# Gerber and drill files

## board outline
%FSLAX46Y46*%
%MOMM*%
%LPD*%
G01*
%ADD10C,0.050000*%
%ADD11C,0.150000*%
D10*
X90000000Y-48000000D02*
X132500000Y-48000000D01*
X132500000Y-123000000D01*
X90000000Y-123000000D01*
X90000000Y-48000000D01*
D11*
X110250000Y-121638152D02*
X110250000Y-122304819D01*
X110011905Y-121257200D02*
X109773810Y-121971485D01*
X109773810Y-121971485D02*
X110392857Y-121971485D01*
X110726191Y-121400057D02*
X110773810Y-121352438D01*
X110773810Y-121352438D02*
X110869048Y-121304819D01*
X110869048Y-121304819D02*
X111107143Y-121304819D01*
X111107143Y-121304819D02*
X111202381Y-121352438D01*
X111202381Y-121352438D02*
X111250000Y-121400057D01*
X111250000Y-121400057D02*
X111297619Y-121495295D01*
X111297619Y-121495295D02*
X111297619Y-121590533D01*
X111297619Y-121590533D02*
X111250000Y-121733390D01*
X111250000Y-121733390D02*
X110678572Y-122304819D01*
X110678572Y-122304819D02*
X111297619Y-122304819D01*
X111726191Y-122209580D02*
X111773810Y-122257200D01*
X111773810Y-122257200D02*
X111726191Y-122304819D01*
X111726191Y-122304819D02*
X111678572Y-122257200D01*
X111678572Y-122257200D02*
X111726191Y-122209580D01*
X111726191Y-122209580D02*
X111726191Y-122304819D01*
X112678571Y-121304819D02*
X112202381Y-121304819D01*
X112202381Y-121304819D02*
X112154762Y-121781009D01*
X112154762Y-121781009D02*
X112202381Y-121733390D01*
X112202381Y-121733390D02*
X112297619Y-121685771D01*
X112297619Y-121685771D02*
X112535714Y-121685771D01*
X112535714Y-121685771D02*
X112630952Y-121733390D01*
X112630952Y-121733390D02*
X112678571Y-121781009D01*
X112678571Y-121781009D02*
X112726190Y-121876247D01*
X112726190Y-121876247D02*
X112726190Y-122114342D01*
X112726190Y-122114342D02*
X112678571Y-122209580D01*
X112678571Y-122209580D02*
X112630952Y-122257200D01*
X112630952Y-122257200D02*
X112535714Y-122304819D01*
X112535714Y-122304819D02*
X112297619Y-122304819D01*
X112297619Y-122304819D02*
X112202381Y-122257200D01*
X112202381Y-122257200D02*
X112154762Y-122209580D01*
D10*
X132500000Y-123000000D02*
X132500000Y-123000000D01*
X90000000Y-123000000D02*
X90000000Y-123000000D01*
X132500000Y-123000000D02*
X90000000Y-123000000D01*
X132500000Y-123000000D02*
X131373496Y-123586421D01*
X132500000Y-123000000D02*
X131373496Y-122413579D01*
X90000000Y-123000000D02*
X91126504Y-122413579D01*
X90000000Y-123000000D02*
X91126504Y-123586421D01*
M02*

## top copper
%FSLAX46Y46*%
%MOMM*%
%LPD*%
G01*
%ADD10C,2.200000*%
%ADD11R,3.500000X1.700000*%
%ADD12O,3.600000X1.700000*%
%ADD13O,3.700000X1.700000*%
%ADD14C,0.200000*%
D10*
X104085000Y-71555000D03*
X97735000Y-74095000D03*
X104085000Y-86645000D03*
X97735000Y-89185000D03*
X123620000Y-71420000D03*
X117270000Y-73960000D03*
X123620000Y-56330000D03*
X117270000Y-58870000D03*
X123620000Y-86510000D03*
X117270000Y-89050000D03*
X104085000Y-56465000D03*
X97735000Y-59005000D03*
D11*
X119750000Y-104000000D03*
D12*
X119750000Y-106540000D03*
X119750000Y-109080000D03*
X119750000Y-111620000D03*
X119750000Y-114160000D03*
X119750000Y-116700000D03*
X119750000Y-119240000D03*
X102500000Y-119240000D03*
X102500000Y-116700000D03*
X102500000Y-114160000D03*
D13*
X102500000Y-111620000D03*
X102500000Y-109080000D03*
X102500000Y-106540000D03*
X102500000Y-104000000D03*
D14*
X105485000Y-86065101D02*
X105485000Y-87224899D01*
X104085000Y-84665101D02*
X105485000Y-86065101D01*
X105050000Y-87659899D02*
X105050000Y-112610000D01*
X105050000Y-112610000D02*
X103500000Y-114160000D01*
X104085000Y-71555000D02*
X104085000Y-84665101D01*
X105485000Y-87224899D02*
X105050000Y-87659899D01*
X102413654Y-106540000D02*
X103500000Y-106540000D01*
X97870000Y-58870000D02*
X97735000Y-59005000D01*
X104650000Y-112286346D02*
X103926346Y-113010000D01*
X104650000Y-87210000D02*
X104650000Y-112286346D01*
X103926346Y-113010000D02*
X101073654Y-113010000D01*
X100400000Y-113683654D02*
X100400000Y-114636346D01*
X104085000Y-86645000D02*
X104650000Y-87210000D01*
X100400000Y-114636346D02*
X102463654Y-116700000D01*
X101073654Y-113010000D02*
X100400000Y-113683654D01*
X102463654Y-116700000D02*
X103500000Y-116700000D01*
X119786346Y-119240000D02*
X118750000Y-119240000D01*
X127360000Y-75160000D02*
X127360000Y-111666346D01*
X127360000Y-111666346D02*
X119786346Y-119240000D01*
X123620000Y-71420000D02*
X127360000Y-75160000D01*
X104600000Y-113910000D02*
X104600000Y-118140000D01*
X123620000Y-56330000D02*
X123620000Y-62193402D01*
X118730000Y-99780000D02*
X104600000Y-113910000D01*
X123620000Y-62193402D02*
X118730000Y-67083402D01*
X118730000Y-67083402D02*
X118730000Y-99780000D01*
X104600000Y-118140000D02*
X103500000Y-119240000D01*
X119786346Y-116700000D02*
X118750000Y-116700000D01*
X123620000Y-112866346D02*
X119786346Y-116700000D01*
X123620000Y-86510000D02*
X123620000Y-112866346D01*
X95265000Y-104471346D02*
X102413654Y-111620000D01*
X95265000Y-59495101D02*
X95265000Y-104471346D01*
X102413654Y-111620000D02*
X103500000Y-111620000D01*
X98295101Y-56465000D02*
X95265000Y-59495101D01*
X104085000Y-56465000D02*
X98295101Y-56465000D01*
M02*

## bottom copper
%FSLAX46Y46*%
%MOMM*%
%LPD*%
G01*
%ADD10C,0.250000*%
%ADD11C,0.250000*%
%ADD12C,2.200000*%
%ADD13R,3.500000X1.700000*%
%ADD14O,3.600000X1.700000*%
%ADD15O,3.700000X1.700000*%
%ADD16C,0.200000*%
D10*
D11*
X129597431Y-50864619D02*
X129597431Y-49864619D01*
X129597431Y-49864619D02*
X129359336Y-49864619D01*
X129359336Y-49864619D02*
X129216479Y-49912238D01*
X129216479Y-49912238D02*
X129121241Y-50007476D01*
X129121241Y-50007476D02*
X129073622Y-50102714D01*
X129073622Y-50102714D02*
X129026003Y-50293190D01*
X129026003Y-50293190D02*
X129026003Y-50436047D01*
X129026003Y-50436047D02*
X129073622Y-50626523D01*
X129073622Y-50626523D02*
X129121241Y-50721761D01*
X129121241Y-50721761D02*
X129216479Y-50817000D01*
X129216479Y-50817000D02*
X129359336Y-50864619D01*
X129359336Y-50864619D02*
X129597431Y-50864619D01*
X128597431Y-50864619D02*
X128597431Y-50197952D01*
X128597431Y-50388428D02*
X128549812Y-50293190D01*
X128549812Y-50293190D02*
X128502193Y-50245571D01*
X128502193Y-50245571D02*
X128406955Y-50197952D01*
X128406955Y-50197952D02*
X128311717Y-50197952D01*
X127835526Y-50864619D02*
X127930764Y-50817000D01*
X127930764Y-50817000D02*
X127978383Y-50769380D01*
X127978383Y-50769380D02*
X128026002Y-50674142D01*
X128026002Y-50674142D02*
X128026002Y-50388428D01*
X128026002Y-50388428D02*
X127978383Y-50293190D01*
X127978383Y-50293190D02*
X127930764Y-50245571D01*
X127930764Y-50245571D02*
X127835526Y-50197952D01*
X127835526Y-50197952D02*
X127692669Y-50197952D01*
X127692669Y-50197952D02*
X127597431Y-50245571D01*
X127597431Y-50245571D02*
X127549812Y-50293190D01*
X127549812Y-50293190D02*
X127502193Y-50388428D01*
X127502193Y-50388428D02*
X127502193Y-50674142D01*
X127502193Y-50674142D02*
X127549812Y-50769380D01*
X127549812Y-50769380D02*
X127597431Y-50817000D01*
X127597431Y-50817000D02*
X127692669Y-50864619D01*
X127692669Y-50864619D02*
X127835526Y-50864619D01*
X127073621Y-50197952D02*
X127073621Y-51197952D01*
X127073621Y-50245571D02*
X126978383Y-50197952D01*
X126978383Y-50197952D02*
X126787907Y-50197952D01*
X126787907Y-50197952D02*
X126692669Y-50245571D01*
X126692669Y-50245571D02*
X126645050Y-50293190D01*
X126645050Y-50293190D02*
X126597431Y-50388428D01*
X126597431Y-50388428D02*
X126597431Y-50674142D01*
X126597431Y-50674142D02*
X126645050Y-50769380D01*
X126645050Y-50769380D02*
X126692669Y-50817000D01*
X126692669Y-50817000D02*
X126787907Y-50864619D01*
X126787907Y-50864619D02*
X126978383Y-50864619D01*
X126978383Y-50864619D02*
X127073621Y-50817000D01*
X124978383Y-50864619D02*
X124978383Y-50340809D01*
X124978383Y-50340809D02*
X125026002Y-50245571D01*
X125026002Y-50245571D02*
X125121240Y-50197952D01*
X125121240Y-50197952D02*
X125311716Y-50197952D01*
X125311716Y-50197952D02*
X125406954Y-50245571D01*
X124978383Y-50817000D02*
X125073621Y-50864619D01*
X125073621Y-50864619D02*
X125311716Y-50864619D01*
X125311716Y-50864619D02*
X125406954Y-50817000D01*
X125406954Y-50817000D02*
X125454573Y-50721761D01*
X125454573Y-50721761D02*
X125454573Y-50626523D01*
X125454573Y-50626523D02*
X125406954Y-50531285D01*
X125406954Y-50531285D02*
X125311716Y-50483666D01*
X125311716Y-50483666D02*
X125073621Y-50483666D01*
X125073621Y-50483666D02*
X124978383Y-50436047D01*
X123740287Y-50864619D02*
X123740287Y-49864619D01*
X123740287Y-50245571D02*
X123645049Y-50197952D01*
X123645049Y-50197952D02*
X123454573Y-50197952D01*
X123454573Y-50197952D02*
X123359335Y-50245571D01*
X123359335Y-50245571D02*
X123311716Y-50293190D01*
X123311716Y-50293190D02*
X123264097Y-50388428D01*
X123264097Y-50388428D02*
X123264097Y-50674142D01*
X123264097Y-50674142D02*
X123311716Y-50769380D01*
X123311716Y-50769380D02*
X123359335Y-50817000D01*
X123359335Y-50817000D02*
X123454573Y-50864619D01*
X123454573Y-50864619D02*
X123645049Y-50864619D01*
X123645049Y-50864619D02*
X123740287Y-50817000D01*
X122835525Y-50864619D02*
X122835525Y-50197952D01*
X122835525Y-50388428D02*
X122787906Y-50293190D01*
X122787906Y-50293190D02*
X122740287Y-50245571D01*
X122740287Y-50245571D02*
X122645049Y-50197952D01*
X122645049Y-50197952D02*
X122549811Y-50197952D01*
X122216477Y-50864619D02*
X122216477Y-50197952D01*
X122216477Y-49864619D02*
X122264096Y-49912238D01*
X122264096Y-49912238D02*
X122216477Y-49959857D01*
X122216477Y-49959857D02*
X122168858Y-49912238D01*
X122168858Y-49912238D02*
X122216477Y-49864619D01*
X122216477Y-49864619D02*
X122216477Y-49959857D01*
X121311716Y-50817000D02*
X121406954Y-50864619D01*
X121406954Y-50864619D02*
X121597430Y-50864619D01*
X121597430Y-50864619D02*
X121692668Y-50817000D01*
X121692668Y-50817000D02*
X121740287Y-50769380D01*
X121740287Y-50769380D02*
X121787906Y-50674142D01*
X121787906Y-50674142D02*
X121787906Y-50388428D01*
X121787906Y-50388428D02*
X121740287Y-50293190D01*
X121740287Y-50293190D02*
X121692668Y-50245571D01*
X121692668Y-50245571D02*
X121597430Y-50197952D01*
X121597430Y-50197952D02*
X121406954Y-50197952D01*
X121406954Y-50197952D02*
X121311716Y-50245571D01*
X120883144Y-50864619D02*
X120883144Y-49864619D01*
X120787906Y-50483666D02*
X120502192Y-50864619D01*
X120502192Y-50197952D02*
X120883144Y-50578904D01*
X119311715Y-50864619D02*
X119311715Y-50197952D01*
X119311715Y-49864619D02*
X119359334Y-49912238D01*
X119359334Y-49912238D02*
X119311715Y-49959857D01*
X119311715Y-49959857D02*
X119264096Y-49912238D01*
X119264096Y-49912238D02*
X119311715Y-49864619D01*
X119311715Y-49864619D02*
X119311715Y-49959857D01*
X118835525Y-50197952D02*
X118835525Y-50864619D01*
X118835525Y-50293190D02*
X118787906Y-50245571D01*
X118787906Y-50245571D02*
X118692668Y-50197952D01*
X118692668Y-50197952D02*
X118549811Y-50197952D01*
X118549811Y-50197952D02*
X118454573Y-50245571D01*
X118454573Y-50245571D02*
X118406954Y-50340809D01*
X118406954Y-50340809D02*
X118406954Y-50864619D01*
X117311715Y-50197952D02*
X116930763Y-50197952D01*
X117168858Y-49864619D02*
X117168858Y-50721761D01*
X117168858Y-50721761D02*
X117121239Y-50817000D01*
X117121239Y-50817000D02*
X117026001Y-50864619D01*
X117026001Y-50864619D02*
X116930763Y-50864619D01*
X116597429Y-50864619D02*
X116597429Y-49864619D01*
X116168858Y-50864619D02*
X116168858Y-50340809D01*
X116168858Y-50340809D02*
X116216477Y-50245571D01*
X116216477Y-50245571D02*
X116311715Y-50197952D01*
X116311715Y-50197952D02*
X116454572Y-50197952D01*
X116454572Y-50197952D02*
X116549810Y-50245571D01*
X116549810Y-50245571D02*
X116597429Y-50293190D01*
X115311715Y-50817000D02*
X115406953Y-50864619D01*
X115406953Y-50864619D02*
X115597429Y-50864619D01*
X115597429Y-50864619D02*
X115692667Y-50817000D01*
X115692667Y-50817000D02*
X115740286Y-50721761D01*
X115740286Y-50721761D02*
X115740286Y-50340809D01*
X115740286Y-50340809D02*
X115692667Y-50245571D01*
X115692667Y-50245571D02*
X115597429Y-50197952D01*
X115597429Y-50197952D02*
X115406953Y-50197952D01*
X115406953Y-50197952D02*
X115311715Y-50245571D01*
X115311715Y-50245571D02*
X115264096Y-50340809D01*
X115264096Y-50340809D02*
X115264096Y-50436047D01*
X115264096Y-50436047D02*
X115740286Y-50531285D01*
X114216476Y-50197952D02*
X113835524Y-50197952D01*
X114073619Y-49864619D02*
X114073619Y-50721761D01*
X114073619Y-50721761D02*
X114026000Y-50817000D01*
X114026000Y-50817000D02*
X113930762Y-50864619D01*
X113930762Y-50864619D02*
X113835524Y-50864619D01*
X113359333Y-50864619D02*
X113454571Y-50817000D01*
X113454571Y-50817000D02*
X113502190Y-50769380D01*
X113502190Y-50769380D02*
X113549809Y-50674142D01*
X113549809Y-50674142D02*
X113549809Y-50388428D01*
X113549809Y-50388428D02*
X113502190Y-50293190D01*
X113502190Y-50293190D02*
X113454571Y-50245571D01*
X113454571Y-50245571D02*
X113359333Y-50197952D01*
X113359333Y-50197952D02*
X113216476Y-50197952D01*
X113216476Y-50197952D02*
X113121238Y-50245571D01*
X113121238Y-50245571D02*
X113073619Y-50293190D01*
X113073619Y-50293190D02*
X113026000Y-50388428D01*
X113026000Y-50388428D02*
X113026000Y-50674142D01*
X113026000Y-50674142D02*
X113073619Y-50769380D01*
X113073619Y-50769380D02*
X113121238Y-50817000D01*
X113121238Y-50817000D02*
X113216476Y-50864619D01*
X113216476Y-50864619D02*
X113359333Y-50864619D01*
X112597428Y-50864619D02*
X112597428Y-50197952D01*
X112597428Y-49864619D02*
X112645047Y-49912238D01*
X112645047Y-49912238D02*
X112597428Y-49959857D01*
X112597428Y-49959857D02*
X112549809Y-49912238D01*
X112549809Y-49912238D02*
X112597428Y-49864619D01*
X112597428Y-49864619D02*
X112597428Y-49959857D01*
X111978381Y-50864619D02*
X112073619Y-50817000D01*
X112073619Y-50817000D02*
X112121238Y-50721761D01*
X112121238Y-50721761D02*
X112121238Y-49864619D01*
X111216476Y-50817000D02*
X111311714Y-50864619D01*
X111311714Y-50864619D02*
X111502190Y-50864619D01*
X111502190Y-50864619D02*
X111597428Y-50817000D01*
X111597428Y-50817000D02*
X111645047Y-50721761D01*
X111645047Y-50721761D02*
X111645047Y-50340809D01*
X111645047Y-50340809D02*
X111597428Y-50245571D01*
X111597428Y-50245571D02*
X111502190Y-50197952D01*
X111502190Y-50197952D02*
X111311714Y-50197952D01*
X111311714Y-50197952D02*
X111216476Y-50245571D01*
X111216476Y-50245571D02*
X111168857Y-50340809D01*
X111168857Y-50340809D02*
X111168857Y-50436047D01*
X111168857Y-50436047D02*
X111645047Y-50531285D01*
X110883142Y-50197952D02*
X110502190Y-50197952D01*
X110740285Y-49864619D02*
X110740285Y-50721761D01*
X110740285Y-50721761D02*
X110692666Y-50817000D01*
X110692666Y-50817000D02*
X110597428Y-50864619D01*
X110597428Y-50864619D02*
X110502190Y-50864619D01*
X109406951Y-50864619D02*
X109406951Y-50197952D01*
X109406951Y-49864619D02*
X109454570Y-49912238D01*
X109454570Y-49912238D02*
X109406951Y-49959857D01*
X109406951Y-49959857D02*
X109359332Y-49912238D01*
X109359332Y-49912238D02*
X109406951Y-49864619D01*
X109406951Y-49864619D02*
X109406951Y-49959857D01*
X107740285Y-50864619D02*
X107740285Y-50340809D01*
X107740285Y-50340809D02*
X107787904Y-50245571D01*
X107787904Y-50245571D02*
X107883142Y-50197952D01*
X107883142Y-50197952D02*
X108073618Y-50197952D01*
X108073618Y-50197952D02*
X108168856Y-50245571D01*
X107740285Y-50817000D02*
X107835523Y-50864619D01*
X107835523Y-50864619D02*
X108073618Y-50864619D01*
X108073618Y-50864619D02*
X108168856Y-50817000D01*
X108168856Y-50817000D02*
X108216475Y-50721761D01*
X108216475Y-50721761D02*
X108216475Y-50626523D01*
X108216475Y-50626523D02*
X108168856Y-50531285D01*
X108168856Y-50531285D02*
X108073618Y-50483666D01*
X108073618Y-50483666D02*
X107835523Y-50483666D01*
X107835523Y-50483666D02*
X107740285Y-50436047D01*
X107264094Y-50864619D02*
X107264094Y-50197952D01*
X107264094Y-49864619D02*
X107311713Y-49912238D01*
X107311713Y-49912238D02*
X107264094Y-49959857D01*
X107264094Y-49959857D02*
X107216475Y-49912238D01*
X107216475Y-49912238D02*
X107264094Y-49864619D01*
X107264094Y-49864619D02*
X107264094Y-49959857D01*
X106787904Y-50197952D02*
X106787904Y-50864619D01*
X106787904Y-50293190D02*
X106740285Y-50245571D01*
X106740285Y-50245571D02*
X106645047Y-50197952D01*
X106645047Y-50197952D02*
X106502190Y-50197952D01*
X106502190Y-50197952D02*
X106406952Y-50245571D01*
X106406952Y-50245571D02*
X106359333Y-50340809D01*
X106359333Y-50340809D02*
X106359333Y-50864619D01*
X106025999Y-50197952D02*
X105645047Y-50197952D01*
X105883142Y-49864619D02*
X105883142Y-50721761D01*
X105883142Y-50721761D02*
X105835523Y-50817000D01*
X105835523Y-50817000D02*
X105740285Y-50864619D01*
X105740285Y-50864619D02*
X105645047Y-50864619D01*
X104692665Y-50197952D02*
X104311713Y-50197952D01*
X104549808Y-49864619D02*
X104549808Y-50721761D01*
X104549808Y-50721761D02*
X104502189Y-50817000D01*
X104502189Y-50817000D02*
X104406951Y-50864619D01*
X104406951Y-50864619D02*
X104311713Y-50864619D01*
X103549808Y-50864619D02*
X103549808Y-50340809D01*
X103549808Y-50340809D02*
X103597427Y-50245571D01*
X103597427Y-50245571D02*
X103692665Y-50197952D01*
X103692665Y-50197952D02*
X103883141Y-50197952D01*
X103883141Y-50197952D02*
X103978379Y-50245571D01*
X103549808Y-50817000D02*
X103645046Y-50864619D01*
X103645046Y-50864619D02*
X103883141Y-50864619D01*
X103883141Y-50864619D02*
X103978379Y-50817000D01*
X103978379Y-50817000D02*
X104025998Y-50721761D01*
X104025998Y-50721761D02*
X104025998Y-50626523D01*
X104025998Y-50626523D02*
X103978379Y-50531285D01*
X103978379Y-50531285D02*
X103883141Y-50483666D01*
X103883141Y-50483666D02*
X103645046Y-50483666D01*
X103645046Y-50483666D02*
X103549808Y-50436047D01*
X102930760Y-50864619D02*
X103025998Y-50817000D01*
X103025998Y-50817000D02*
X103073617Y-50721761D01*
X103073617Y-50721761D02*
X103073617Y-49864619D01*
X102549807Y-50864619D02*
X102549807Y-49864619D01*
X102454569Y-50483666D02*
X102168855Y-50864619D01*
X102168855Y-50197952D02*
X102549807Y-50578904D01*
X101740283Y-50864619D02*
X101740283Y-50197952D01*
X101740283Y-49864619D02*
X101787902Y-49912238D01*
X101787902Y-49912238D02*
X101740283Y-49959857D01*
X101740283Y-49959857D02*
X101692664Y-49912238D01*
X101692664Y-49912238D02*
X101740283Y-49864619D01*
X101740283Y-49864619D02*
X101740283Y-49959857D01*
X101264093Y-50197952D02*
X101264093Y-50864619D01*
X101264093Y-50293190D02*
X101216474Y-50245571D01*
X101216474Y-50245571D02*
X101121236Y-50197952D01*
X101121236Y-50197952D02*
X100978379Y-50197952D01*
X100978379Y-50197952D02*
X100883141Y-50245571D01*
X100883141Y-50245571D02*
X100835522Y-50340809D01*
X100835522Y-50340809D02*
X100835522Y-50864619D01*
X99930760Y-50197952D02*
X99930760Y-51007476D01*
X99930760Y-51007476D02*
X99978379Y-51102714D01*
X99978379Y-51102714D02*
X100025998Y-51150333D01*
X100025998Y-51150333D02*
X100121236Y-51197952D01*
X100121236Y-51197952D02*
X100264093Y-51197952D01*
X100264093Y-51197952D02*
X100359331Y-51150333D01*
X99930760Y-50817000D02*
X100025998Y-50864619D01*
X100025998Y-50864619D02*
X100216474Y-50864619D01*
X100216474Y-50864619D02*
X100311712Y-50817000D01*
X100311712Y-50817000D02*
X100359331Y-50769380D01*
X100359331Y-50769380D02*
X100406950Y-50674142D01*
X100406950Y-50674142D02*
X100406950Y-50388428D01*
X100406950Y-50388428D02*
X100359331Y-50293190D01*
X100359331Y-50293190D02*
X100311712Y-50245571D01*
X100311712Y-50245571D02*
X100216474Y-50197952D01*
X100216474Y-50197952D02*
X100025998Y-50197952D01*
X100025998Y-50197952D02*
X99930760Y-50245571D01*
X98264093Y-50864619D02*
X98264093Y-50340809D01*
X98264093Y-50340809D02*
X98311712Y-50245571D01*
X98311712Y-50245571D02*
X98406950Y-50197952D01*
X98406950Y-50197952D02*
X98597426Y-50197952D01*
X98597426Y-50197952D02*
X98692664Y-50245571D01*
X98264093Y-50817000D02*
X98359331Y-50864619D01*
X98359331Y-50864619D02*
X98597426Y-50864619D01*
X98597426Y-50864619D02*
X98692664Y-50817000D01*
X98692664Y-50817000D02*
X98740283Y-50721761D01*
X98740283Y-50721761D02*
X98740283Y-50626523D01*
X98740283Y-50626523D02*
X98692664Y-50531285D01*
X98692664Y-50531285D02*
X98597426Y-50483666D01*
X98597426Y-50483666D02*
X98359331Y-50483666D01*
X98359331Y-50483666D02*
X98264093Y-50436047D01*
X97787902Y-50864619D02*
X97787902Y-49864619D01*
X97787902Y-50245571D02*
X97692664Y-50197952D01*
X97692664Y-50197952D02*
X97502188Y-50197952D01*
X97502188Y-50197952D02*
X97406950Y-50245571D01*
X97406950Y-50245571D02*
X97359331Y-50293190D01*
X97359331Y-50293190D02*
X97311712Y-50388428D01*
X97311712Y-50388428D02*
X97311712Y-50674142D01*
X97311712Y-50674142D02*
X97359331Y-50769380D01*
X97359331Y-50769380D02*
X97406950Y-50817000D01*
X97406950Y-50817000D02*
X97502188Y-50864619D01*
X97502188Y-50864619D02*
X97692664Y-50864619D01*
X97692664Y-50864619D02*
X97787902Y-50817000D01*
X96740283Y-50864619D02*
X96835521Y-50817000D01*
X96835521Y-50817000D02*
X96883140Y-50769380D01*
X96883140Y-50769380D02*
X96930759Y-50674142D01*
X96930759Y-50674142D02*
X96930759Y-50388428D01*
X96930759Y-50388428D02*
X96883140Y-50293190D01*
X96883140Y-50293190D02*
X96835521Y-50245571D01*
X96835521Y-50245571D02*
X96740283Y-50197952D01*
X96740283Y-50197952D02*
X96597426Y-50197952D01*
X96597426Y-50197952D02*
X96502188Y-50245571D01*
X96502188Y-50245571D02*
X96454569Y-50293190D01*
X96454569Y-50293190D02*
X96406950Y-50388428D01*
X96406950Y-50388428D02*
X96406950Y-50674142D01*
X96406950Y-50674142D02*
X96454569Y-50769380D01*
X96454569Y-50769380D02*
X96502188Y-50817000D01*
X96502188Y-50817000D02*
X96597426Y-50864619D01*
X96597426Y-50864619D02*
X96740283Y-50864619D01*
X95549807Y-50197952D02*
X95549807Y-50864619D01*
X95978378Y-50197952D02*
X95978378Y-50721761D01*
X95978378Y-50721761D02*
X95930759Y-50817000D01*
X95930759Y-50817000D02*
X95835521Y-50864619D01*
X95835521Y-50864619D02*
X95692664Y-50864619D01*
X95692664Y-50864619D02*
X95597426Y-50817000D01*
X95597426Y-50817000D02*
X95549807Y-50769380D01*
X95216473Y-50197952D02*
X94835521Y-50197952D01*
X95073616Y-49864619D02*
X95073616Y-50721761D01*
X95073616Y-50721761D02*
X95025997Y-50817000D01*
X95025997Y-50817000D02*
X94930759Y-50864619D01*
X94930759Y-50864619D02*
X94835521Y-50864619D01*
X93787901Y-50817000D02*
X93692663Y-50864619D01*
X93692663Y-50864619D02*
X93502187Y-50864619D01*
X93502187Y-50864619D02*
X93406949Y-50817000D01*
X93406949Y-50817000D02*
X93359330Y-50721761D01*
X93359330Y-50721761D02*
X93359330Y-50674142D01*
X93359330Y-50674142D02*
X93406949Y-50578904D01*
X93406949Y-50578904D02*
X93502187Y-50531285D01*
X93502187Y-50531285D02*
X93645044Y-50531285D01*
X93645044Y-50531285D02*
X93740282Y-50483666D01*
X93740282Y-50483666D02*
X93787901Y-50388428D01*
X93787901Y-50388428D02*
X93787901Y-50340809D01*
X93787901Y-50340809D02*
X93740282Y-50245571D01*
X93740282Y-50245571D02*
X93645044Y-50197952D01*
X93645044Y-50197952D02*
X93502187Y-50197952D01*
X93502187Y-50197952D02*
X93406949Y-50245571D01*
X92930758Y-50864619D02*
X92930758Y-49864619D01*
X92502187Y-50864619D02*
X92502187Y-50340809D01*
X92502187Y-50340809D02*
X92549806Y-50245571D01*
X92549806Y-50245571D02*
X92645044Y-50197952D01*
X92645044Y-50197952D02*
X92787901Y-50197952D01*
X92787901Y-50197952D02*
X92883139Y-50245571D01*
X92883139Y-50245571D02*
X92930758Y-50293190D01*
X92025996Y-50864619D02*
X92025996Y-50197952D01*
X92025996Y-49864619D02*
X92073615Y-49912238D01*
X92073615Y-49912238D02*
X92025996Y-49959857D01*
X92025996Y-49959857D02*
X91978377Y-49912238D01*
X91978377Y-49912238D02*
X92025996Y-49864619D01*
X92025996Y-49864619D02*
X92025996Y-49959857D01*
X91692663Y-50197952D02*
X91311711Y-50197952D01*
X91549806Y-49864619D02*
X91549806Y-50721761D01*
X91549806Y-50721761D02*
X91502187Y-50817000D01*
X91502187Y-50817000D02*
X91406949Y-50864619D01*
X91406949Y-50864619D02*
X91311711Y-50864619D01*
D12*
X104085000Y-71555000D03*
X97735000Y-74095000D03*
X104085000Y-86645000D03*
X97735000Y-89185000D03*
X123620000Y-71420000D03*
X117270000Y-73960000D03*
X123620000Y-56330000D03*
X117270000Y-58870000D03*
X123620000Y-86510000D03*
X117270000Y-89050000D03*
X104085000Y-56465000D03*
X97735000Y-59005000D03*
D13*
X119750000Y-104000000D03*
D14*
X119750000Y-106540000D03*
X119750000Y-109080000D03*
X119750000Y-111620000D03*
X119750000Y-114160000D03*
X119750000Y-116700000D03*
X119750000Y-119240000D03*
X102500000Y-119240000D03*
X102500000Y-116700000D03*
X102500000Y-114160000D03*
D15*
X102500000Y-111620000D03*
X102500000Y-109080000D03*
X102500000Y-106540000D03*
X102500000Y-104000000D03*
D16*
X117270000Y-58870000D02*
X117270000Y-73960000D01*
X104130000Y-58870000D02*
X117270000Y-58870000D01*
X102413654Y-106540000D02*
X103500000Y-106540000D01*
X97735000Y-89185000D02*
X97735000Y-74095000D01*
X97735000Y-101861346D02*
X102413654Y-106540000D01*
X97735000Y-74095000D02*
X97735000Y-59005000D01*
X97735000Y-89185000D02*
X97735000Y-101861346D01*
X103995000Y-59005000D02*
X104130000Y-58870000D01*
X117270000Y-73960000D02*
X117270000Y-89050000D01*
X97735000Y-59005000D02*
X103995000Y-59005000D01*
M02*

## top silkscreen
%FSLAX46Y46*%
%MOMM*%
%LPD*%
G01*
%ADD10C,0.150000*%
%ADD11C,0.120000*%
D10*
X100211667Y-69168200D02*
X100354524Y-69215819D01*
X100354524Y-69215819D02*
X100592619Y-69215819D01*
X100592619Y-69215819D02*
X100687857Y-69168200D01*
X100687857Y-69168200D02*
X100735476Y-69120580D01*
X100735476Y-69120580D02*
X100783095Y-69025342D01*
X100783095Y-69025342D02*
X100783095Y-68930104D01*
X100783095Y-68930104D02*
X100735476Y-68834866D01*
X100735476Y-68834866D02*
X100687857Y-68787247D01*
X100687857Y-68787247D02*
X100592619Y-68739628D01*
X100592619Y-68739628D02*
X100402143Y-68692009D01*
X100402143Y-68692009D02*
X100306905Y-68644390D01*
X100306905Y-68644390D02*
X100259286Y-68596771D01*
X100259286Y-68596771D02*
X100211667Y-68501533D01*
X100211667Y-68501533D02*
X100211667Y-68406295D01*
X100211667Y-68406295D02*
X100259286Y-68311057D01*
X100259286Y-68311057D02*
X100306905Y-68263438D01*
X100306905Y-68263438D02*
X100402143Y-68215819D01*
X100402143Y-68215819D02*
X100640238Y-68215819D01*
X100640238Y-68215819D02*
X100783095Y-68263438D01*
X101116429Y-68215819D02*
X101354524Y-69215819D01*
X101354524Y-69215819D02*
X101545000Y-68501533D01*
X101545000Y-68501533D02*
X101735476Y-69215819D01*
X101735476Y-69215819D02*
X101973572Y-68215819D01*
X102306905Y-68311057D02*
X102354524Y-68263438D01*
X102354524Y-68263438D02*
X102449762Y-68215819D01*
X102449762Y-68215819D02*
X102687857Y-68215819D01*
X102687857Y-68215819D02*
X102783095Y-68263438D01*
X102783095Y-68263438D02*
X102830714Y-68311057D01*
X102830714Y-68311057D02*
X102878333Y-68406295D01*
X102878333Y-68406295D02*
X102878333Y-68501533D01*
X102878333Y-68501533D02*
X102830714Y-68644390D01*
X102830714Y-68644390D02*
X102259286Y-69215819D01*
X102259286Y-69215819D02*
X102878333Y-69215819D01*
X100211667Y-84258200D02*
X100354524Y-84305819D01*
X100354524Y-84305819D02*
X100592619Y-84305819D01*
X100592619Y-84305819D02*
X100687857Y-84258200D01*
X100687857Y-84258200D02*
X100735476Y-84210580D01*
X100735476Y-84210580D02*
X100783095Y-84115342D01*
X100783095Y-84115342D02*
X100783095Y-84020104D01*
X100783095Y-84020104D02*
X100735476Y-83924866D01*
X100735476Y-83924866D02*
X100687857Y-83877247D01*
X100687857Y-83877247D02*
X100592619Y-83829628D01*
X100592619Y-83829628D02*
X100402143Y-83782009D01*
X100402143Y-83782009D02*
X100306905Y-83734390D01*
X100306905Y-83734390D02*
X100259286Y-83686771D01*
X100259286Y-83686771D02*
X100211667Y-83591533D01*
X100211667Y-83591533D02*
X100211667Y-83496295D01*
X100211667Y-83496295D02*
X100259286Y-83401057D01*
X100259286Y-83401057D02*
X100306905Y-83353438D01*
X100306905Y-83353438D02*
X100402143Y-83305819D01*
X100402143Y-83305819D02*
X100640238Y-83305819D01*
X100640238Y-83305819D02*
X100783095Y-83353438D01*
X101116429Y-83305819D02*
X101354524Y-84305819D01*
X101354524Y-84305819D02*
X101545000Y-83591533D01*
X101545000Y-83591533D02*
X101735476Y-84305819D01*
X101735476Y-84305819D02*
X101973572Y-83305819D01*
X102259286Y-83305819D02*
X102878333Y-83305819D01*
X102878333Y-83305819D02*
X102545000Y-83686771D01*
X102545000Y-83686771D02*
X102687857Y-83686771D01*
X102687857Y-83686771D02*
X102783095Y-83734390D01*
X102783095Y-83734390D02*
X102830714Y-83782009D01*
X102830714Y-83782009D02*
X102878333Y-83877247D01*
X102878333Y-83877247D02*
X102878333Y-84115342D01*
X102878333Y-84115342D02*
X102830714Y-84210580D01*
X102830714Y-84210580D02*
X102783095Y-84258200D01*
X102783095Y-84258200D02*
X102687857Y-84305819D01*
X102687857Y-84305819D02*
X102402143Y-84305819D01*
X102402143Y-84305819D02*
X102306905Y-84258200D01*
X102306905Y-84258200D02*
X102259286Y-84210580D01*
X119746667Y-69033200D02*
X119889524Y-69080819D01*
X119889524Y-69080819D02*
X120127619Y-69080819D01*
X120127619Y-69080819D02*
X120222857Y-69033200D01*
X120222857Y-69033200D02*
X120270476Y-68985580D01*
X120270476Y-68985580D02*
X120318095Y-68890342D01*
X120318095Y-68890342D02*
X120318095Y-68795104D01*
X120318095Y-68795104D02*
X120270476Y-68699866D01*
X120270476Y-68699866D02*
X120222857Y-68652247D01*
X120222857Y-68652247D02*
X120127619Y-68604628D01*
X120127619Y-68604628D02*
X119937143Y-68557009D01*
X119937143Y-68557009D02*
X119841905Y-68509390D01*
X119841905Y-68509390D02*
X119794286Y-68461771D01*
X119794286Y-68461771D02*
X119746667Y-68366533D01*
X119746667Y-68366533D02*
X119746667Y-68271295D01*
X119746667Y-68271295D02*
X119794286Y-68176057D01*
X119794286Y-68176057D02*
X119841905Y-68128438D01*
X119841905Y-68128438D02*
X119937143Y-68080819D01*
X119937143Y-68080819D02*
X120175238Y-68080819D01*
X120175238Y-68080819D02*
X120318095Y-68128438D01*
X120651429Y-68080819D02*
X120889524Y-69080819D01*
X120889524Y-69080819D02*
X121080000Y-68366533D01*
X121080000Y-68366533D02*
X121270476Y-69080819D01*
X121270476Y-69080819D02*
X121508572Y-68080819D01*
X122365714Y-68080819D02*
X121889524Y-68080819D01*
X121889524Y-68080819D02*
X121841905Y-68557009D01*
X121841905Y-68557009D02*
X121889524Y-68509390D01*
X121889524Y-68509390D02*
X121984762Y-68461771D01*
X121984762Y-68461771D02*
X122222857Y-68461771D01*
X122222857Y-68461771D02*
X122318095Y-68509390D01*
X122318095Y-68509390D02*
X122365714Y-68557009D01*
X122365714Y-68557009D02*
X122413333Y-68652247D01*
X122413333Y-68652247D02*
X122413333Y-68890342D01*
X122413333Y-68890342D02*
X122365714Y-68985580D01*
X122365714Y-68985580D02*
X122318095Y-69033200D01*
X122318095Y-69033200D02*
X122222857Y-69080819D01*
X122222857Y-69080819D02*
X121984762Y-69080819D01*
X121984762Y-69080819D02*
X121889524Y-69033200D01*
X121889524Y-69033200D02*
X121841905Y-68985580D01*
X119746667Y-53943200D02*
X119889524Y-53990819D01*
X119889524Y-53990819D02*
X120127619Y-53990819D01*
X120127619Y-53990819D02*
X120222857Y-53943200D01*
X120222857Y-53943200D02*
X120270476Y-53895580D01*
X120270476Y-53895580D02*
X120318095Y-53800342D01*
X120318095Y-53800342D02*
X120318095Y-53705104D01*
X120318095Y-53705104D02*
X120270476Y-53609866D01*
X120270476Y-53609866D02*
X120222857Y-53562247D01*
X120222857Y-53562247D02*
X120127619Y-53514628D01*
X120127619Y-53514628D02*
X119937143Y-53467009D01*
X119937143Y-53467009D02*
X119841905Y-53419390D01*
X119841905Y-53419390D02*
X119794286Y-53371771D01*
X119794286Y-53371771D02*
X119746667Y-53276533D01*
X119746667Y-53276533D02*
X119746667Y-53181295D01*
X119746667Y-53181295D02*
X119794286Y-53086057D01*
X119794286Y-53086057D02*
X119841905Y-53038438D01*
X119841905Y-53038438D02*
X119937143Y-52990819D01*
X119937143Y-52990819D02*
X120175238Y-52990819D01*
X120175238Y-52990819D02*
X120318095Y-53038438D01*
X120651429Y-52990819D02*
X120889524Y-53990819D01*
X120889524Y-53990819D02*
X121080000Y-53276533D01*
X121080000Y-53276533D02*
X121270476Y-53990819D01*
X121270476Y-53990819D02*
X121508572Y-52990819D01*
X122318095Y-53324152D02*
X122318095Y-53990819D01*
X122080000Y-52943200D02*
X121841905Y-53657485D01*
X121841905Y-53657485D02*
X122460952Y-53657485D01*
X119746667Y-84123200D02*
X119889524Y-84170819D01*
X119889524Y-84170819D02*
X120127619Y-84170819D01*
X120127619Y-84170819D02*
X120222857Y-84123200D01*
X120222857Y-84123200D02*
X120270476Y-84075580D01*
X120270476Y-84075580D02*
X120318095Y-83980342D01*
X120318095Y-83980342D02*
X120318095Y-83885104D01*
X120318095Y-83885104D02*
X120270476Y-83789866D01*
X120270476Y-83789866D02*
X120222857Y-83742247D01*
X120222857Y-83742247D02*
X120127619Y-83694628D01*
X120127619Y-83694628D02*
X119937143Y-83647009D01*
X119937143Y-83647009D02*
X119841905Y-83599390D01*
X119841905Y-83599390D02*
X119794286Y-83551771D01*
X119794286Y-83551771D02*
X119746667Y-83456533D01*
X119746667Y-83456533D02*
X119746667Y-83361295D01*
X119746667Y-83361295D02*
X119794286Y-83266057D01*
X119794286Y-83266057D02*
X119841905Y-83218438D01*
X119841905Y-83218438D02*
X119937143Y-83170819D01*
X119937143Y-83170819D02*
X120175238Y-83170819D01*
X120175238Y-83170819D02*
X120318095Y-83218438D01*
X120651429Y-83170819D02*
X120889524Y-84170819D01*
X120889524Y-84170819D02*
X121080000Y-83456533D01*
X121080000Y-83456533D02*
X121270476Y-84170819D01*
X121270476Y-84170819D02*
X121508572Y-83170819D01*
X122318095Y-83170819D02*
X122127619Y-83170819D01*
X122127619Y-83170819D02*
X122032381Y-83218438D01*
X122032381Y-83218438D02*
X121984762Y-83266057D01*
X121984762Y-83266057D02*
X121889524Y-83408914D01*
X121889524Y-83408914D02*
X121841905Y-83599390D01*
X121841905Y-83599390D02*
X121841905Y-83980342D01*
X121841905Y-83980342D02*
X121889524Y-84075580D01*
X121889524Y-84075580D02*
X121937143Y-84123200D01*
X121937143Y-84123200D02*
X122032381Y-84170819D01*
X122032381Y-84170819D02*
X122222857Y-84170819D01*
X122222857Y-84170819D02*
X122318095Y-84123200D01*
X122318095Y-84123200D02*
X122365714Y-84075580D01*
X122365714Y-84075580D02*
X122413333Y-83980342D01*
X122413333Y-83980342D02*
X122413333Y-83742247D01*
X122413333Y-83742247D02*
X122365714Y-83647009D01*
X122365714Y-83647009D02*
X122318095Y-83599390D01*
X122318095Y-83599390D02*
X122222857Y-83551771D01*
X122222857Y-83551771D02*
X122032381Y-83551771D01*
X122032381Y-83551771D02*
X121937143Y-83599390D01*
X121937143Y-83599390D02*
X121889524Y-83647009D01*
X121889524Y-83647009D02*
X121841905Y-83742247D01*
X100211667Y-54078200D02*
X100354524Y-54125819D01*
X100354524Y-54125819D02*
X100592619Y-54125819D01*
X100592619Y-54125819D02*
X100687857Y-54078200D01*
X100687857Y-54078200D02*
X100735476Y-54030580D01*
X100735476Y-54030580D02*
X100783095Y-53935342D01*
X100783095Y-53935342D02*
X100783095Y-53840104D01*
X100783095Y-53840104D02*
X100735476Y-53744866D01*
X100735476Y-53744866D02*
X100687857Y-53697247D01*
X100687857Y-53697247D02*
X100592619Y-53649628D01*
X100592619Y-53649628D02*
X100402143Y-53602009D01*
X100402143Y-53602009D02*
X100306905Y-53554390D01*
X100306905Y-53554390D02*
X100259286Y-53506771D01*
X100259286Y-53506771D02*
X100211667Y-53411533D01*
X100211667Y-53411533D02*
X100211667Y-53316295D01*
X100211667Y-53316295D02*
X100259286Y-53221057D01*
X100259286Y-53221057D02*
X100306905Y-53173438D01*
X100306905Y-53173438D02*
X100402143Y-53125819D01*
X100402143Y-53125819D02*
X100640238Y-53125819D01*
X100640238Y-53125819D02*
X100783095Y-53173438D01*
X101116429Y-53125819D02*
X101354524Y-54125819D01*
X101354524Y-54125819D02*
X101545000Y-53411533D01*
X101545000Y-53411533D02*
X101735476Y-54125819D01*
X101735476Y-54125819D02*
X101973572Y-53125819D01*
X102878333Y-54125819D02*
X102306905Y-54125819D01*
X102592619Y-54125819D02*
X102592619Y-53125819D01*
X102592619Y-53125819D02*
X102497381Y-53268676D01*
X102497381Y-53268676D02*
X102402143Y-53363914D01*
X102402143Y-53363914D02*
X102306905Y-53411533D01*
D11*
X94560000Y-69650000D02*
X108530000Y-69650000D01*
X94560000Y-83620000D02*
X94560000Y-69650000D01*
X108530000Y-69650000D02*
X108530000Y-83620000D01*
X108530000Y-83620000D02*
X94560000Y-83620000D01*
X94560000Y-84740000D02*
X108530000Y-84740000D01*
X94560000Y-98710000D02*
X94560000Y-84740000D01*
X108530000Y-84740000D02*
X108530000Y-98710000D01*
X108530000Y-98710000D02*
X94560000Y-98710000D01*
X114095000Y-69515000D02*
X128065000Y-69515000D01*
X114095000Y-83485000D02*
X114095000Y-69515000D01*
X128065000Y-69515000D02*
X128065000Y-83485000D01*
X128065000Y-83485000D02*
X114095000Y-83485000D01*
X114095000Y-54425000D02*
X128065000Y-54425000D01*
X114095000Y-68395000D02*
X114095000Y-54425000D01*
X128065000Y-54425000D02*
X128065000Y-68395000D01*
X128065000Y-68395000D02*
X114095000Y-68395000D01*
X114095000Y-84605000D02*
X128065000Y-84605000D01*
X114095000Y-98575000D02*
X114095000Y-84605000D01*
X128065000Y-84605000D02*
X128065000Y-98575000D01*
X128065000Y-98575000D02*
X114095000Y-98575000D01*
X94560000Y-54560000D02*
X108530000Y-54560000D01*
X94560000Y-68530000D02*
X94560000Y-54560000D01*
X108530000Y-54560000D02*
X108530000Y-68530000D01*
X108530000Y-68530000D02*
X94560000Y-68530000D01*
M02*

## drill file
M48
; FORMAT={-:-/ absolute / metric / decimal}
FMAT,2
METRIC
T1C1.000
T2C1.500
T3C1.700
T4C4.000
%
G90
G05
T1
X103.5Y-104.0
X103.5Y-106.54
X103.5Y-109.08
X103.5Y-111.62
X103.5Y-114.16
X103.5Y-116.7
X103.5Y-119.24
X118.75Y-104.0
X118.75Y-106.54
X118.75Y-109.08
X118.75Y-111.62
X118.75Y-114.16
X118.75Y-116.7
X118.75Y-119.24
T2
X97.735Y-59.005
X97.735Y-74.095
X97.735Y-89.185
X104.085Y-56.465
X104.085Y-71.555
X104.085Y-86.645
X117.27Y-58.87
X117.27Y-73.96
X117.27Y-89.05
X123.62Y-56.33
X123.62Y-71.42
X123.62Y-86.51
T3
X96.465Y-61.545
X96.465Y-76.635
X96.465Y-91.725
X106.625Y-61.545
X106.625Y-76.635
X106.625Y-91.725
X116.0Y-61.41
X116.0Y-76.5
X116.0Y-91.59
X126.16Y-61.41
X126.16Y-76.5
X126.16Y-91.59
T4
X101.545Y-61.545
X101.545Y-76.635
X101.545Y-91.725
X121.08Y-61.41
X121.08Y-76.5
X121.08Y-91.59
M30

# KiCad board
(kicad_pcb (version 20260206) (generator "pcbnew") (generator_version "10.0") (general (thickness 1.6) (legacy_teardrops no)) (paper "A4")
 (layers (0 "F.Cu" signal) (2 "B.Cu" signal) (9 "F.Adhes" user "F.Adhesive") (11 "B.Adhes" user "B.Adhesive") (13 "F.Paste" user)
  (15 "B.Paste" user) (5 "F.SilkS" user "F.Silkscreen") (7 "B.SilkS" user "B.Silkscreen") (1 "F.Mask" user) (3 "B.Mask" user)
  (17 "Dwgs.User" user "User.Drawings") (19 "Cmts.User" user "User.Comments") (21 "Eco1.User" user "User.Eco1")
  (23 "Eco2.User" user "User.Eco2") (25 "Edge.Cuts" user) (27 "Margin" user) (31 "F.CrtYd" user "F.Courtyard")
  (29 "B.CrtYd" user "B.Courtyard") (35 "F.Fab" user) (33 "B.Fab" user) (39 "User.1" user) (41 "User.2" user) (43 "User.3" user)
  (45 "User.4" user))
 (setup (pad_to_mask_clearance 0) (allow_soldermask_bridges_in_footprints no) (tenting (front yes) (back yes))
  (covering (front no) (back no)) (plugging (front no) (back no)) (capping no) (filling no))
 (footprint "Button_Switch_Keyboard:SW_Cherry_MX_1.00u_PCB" (layer "F.Cu") (at 104.085 71.555)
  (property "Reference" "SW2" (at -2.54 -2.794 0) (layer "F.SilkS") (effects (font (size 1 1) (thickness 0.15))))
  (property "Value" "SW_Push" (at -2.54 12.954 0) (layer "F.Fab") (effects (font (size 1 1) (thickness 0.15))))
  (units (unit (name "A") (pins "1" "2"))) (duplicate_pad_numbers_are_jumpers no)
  (fp_line (start -9.525 -1.905) (end 4.445 -1.905) (stroke (width 0.12) (type solid)) (layer "F.SilkS"))
  (fp_line (start -9.525 12.065) (end -9.525 -1.905) (stroke (width 0.12) (type solid)) (layer "F.SilkS"))
  (fp_line (start 4.445 -1.905) (end 4.445 12.065) (stroke (width 0.12) (type solid)) (layer "F.SilkS"))
  (fp_line (start 4.445 12.065) (end -9.525 12.065) (stroke (width 0.12) (type solid)) (layer "F.SilkS"))
  (pad "" np_thru_hole circle (at -7.62 5.08) (size 1.7 1.7) (drill 1.7) (layers "*.Cu" "*.Mask"))
  (pad "" np_thru_hole circle (at -2.54 5.08) (size 4 4) (drill 4) (layers "*.Cu" "*.Mask"))
  (pad "" np_thru_hole circle (at 2.54 5.08) (size 1.7 1.7) (drill 1.7) (layers "*.Cu" "*.Mask"))
  (pad "1" thru_hole circle (at 0 0) (size 2.2 2.2) (drill 1.5) (layers "*.Cu" "*.Mask") (remove_unused_layers no)
   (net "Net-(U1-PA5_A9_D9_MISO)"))
  (pad "2" thru_hole circle (at -6.35 2.54) (size 2.2 2.2) (drill 1.5) (layers "*.Cu" "*.Mask") (remove_unused_layers no) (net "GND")))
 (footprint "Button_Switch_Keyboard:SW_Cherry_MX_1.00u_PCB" (layer "F.Cu") (at 104.085 86.645)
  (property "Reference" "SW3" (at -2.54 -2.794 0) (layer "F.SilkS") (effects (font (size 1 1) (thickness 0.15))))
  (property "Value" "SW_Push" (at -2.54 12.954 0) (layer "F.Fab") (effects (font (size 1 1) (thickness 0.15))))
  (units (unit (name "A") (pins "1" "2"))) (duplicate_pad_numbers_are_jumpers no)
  (fp_line (start -9.525 -1.905) (end 4.445 -1.905) (stroke (width 0.12) (type solid)) (layer "F.SilkS"))
  (fp_line (start -9.525 12.065) (end -9.525 -1.905) (stroke (width 0.12) (type solid)) (layer "F.SilkS"))
  (fp_line (start 4.445 -1.905) (end 4.445 12.065) (stroke (width 0.12) (type solid)) (layer "F.SilkS"))
  (fp_line (start 4.445 12.065) (end -9.525 12.065) (stroke (width 0.12) (type solid)) (layer "F.SilkS"))
  (pad "" np_thru_hole circle (at -7.62 5.08) (size 1.7 1.7) (drill 1.7) (layers "*.Cu" "*.Mask"))
  (pad "" np_thru_hole circle (at -2.54 5.08) (size 4 4) (drill 4) (layers "*.Cu" "*.Mask"))
  (pad "" np_thru_hole circle (at 2.54 5.08) (size 1.7 1.7) (drill 1.7) (layers "*.Cu" "*.Mask"))
  (pad "1" thru_hole circle (at 0 0) (size 2.2 2.2) (drill 1.5) (layers "*.Cu" "*.Mask") (remove_unused_layers no)
   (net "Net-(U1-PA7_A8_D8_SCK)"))
  (pad "2" thru_hole circle (at -6.35 2.54) (size 2.2 2.2) (drill 1.5) (layers "*.Cu" "*.Mask") (remove_unused_layers no) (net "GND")))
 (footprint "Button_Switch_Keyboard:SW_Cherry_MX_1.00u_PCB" (layer "F.Cu") (at 123.62 71.42)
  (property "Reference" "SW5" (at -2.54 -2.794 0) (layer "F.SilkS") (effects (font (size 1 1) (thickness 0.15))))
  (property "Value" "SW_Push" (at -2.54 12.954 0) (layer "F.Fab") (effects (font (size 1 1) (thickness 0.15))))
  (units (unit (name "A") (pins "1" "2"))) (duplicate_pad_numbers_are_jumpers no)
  (fp_line (start -9.525 -1.905) (end 4.445 -1.905) (stroke (width 0.12) (type solid)) (layer "F.SilkS"))
  (fp_line (start -9.525 12.065) (end -9.525 -1.905) (stroke (width 0.12) (type solid)) (layer "F.SilkS"))
  (fp_line (start 4.445 -1.905) (end 4.445 12.065) (stroke (width 0.12) (type solid)) (layer "F.SilkS"))
  (fp_line (start 4.445 12.065) (end -9.525 12.065) (stroke (width 0.12) (type solid)) (layer "F.SilkS"))
  (pad "" np_thru_hole circle (at -7.62 5.08) (size 1.7 1.7) (drill 1.7) (layers "*.Cu" "*.Mask"))
  (pad "" np_thru_hole circle (at -2.54 5.08) (size 4 4) (drill 4) (layers "*.Cu" "*.Mask"))
  (pad "" np_thru_hole circle (at 2.54 5.08) (size 1.7 1.7) (drill 1.7) (layers "*.Cu" "*.Mask"))
  (pad "1" thru_hole circle (at 0 0) (size 2.2 2.2) (drill 1.5) (layers "*.Cu" "*.Mask") (remove_unused_layers no)
   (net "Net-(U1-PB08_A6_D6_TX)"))
  (pad "2" thru_hole circle (at -6.35 2.54) (size 2.2 2.2) (drill 1.5) (layers "*.Cu" "*.Mask") (remove_unused_layers no) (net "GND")))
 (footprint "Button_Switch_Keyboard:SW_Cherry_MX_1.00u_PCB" (layer "F.Cu") (at 123.62 56.33)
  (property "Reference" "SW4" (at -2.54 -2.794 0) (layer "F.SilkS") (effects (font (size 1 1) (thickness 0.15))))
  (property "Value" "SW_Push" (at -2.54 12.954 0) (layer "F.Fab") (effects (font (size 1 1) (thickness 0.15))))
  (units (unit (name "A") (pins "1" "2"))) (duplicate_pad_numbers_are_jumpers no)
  (fp_line (start -9.525 -1.905) (end 4.445 -1.905) (stroke (width 0.12) (type solid)) (layer "F.SilkS"))
  (fp_line (start -9.525 12.065) (end -9.525 -1.905) (stroke (width 0.12) (type solid)) (layer "F.SilkS"))
  (fp_line (start 4.445 -1.905) (end 4.445 12.065) (stroke (width 0.12) (type solid)) (layer "F.SilkS"))
  (fp_line (start 4.445 12.065) (end -9.525 12.065) (stroke (width 0.12) (type solid)) (layer "F.SilkS"))
  (pad "" np_thru_hole circle (at -7.62 5.08) (size 1.7 1.7) (drill 1.7) (layers "*.Cu" "*.Mask"))
  (pad "" np_thru_hole circle (at -2.54 5.08) (size 4 4) (drill 4) (layers "*.Cu" "*.Mask"))
  (pad "" np_thru_hole circle (at 2.54 5.08) (size 1.7 1.7) (drill 1.7) (layers "*.Cu" "*.Mask"))
  (pad "1" thru_hole circle (at 0 0) (size 2.2 2.2) (drill 1.5) (layers "*.Cu" "*.Mask") (remove_unused_layers no)
   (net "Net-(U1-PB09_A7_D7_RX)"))
  (pad "2" thru_hole circle (at -6.35 2.54) (size 2.2 2.2) (drill 1.5) (layers "*.Cu" "*.Mask") (remove_unused_layers no) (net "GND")))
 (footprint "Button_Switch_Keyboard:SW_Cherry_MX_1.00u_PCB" (layer "F.Cu") (at 123.62 86.51)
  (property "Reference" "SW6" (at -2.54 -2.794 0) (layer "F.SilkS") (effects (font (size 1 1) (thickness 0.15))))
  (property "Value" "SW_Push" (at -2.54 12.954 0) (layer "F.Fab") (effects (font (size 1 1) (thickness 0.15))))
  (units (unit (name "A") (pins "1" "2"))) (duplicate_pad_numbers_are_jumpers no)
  (fp_line (start -9.525 -1.905) (end 4.445 -1.905) (stroke (width 0.12) (type solid)) (layer "F.SilkS"))
  (fp_line (start -9.525 12.065) (end -9.525 -1.905) (stroke (width 0.12) (type solid)) (layer "F.SilkS"))
  (fp_line (start 4.445 -1.905) (end 4.445 12.065) (stroke (width 0.12) (type solid)) (layer "F.SilkS"))
  (fp_line (start 4.445 12.065) (end -9.525 12.065) (stroke (width 0.12) (type solid)) (layer "F.SilkS"))
  (pad "" np_thru_hole circle (at -7.62 5.08) (size 1.7 1.7) (drill 1.7) (layers "*.Cu" "*.Mask"))
  (pad "" np_thru_hole circle (at -2.54 5.08) (size 4 4) (drill 4) (layers "*.Cu" "*.Mask"))
  (pad "" np_thru_hole circle (at 2.54 5.08) (size 1.7 1.7) (drill 1.7) (layers "*.Cu" "*.Mask"))
  (pad "1" thru_hole circle (at 0 0) (size 2.2 2.2) (drill 1.5) (layers "*.Cu" "*.Mask") (remove_unused_layers no)
   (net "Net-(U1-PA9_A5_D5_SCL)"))
  (pad "2" thru_hole circle (at -6.35 2.54) (size 2.2 2.2) (drill 1.5) (layers "*.Cu" "*.Mask") (remove_unused_layers no) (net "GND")))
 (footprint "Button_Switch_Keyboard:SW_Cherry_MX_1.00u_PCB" (layer "F.Cu") (at 104.085 56.465)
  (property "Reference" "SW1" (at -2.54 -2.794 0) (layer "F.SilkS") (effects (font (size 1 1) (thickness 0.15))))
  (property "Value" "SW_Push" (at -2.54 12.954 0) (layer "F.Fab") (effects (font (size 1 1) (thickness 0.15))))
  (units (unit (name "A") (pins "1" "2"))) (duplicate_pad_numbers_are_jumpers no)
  (fp_line (start -9.525 -1.905) (end 4.445 -1.905) (stroke (width 0.12) (type solid)) (layer "F.SilkS"))
  (fp_line (start -9.525 12.065) (end -9.525 -1.905) (stroke (width 0.12) (type solid)) (layer "F.SilkS"))
  (fp_line (start 4.445 -1.905) (end 4.445 12.065) (stroke (width 0.12) (type solid)) (layer "F.SilkS"))
  (fp_line (start 4.445 12.065) (end -9.525 12.065) (stroke (width 0.12) (type solid)) (layer "F.SilkS"))
  (pad "" np_thru_hole circle (at -7.62 5.08) (size 1.7 1.7) (drill 1.7) (layers "*.Cu" "*.Mask"))
  (pad "" np_thru_hole circle (at -2.54 5.08) (size 4 4) (drill 4) (layers "*.Cu" "*.Mask"))
  (pad "" np_thru_hole circle (at 2.54 5.08) (size 1.7 1.7) (drill 1.7) (layers "*.Cu" "*.Mask"))
  (pad "1" thru_hole circle (at 0 0) (size 2.2 2.2) (drill 1.5) (layers "*.Cu" "*.Mask") (remove_unused_layers no)
   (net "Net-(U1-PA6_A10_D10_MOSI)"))
  (pad "2" thru_hole circle (at -6.35 2.54) (size 2.2 2.2) (drill 1.5) (layers "*.Cu" "*.Mask") (remove_unused_layers no) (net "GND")))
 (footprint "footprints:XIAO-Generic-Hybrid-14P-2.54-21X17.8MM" (layer "B.Cu") (at 111.125 111.62 180)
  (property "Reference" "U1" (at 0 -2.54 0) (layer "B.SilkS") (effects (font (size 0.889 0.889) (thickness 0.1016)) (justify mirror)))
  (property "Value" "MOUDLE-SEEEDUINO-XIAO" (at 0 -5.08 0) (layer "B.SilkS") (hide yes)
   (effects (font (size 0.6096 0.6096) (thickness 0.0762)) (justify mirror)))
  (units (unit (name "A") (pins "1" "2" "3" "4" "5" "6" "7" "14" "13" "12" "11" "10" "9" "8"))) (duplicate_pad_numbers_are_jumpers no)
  (pad "1" thru_hole rect (at -7.625 7.62 180) (size 3.5 1.7) (drill 1 (offset -1 0)) (layers "*.Cu" "*.Mask") (remove_unused_layers no)
   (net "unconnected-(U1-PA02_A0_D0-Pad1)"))
  (pad "2" thru_hole oval (at -7.625 5.08 180) (size 3.6 1.7) (drill 1 (offset -1 0)) (layers "*.Cu" "*.Mask") (remove_unused_layers no)
   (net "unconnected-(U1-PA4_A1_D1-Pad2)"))
  (pad "3" thru_hole oval (at -7.625 2.54 180) (size 3.6 1.7) (drill 1 (offset -1 0)) (layers "*.Cu" "*.Mask") (remove_unused_layers no)
   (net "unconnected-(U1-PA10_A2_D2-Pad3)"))
  (pad "4" thru_hole oval (at -7.625 0 180) (size 3.6 1.7) (drill 1 (offset -1 0)) (layers "*.Cu" "*.Mask") (remove_unused_layers no)
   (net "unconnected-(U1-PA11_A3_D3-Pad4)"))
  (pad "5" thru_hole oval (at -7.625 -2.54 180) (size 3.6 1.7) (drill 1 (offset -1 0)) (layers "*.Cu" "*.Mask") (remove_unused_layers no)
   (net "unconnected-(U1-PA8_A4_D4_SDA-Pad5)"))
  (pad "6" thru_hole oval (at -7.625 -5.08) (size 3.6 1.7) (drill 1 (offset 1 0)) (layers "*.Cu" "*.Mask") (remove_unused_layers no)
   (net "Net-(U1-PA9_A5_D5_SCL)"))
  (pad "7" thru_hole oval (at -7.625 -7.62 180) (size 3.6 1.7) (drill 1 (offset -1 0)) (layers "*.Cu" "*.Mask") (remove_unused_layers no)
   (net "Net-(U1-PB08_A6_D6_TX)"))
  (pad "8" thru_hole oval (at 7.625 -7.62 180) (size 3.6 1.7) (drill 1 (offset 1 0)) (layers "*.Cu" "*.Mask") (remove_unused_layers no)
   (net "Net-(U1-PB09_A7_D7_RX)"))
  (pad "9" thru_hole oval (at 7.625 -5.08 180) (size 3.6 1.7) (drill 1 (offset 1 0)) (layers "*.Cu" "*.Mask") (remove_unused_layers no)
   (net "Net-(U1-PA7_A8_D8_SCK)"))
  (pad "10" thru_hole oval (at 7.625 -2.54 180) (size 3.6 1.7) (drill 1 (offset 1 0)) (layers "*.Cu" "*.Mask") (remove_unused_layers no)
   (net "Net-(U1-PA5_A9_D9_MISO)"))
  (pad "11" thru_hole oval (at 7.625 0 180) (size 3.7 1.7) (drill 1 (offset 1 0)) (layers "*.Cu" "*.Mask") (remove_unused_layers no)
   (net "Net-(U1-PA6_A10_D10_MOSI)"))
  (pad "12" thru_hole oval (at 7.625 2.54 180) (size 3.7 1.7) (drill 1 (offset 1 0)) (layers "*.Cu" "*.Mask") (remove_unused_layers no)
   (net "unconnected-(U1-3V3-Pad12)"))
  (pad "13" thru_hole oval (at 7.625 5.08 180) (size 3.7 1.7) (drill 1 (offset 1 0)) (layers "*.Cu" "*.Mask") (remove_unused_layers no)
   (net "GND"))
  (pad "14" thru_hole oval (at 7.625 7.62 180) (size 3.7 1.7) (drill 1 (offset 1 0)) (layers "*.Cu" "*.Mask") (remove_unused_layers no)
   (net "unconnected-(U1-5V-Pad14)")))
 (gr_rect (start 90 48) (end 132.5 123) (stroke (width 0.05) (type default)) (fill no) (layer "Edge.Cuts"))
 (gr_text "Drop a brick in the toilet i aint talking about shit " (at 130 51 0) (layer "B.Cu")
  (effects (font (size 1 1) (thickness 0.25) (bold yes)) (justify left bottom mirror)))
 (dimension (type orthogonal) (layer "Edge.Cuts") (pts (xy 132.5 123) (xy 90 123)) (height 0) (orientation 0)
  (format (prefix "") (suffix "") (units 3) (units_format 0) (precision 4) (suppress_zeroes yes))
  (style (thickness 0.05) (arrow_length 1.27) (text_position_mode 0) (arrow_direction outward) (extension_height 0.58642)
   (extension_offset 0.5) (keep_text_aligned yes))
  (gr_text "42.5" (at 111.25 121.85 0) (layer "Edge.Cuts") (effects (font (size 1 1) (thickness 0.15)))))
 (segment (start 105.485 86.065101) (end 105.485 87.224899) (width 0.2) (layer "F.Cu") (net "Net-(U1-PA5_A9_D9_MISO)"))
 (segment (start 104.085 84.665101) (end 105.485 86.065101) (width 0.2) (layer "F.Cu") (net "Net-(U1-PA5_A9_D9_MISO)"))
 (segment (start 105.05 87.659899) (end 105.05 112.61) (width 0.2) (layer "F.Cu") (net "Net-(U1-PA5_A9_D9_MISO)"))
 (segment (start 105.05 112.61) (end 103.5 114.16) (width 0.2) (layer "F.Cu") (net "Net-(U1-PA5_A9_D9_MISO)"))
 (segment (start 104.085 71.555) (end 104.085 84.665101) (width 0.2) (layer "F.Cu") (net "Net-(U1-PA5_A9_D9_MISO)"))
 (segment (start 105.485 87.224899) (end 105.05 87.659899) (width 0.2) (layer "F.Cu") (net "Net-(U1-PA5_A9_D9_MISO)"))
 (segment (start 102.413654 106.54) (end 103.5 106.54) (width 0.2) (layer "F.Cu") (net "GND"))
 (segment (start 97.87 58.87) (end 97.735 59.005) (width 0.2) (layer "F.Cu") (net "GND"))
 (segment (start 117.27 58.87) (end 117.27 73.96) (width 0.2) (layer "B.Cu") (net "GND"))
 (segment (start 104.13 58.87) (end 117.27 58.87) (width 0.2) (layer "B.Cu") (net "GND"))
 (segment (start 102.413654 106.54) (end 103.5 106.54) (width 0.2) (layer "B.Cu") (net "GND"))
 (segment (start 97.735 89.185) (end 97.735 74.095) (width 0.2) (layer "B.Cu") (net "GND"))
 (segment (start 97.735 101.861346) (end 102.413654 106.54) (width 0.2) (layer "B.Cu") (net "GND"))
 (segment (start 97.735 74.095) (end 97.735 59.005) (width 0.2) (layer "B.Cu") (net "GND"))
 (segment (start 97.735 89.185) (end 97.735 101.861346) (width 0.2) (layer "B.Cu") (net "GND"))
 (segment (start 103.995 59.005) (end 104.13 58.87) (width 0.2) (layer "B.Cu") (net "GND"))
 (segment (start 117.27 73.96) (end 117.27 89.05) (width 0.2) (layer "B.Cu") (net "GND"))
 (segment (start 97.735 59.005) (end 103.995 59.005) (width 0.2) (layer "B.Cu") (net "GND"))
 (segment (start 104.65 112.286346) (end 103.926346 113.01) (width 0.2) (layer "F.Cu") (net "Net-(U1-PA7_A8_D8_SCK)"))
 (segment (start 104.65 87.21) (end 104.65 112.286346) (width 0.2) (layer "F.Cu") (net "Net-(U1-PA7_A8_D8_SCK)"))
 (segment (start 103.926346 113.01) (end 101.073654 113.01) (width 0.2) (layer "F.Cu") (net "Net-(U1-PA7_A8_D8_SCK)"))
 (segment (start 100.4 113.683654) (end 100.4 114.636346) (width 0.2) (layer "F.Cu") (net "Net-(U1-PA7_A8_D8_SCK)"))
 (segment (start 104.085 86.645) (end 104.65 87.21) (width 0.2) (layer "F.Cu") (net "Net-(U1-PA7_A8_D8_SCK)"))
 (segment (start 100.4 114.636346) (end 102.463654 116.7) (width 0.2) (layer "F.Cu") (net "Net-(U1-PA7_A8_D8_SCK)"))
 (segment (start 101.073654 113.01) (end 100.4 113.683654) (width 0.2) (layer "F.Cu") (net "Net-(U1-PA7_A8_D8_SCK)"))
 (segment (start 102.463654 116.7) (end 103.5 116.7) (width 0.2) (layer "F.Cu") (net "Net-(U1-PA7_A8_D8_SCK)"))
 (segment (start 119.786346 119.24) (end 118.75 119.24) (width 0.2) (layer "F.Cu") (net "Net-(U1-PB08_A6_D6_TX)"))
 (segment (start 127.36 75.16) (end 127.36 111.666346) (width 0.2) (layer "F.Cu") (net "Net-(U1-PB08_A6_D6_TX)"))
 (segment (start 127.36 111.666346) (end 119.786346 119.24) (width 0.2) (layer "F.Cu") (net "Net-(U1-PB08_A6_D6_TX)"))
 (segment (start 123.62 71.42) (end 127.36 75.16) (width 0.2) (layer "F.Cu") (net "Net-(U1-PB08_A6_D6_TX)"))
 (segment (start 104.6 113.91) (end 104.6 118.14) (width 0.2) (layer "F.Cu") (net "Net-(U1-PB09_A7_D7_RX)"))
 (segment (start 123.62 56.33) (end 123.62 62.193402) (width 0.2) (layer "F.Cu") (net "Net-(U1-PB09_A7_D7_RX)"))
 (segment (start 118.73 99.78) (end 104.6 113.91) (width 0.2) (layer "F.Cu") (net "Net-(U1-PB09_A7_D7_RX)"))
 (segment (start 123.62 62.193402) (end 118.73 67.083402) (width 0.2) (layer "F.Cu") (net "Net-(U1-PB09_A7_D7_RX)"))
 (segment (start 118.73 67.083402) (end 118.73 99.78) (width 0.2) (layer "F.Cu") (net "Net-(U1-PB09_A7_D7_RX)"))
 (segment (start 104.6 118.14) (end 103.5 119.24) (width 0.2) (layer "F.Cu") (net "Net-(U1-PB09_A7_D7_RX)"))
 (segment (start 119.786346 116.7) (end 118.75 116.7) (width 0.2) (layer "F.Cu") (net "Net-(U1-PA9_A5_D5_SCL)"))
 (segment (start 123.62 112.866346) (end 119.786346 116.7) (width 0.2) (layer "F.Cu") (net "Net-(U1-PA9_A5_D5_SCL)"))
 (segment (start 123.62 86.51) (end 123.62 112.866346) (width 0.2) (layer "F.Cu") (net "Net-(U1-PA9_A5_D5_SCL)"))
 (segment (start 95.265 104.471346) (end 102.413654 111.62) (width 0.2) (layer "F.Cu") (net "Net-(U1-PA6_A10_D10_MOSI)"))
 (segment (start 95.265 59.495101) (end 95.265 104.471346) (width 0.2) (layer "F.Cu") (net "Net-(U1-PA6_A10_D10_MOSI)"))
 (segment (start 102.413654 111.62) (end 103.5 111.62) (width 0.2) (layer "F.Cu") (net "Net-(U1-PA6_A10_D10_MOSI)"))
 (segment (start 98.295101 56.465) (end 95.265 59.495101) (width 0.2) (layer "F.Cu") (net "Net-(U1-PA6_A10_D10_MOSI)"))
 (segment (start 104.085 56.465) (end 98.295101 56.465) (width 0.2) (layer "F.Cu") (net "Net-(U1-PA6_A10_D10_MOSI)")))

